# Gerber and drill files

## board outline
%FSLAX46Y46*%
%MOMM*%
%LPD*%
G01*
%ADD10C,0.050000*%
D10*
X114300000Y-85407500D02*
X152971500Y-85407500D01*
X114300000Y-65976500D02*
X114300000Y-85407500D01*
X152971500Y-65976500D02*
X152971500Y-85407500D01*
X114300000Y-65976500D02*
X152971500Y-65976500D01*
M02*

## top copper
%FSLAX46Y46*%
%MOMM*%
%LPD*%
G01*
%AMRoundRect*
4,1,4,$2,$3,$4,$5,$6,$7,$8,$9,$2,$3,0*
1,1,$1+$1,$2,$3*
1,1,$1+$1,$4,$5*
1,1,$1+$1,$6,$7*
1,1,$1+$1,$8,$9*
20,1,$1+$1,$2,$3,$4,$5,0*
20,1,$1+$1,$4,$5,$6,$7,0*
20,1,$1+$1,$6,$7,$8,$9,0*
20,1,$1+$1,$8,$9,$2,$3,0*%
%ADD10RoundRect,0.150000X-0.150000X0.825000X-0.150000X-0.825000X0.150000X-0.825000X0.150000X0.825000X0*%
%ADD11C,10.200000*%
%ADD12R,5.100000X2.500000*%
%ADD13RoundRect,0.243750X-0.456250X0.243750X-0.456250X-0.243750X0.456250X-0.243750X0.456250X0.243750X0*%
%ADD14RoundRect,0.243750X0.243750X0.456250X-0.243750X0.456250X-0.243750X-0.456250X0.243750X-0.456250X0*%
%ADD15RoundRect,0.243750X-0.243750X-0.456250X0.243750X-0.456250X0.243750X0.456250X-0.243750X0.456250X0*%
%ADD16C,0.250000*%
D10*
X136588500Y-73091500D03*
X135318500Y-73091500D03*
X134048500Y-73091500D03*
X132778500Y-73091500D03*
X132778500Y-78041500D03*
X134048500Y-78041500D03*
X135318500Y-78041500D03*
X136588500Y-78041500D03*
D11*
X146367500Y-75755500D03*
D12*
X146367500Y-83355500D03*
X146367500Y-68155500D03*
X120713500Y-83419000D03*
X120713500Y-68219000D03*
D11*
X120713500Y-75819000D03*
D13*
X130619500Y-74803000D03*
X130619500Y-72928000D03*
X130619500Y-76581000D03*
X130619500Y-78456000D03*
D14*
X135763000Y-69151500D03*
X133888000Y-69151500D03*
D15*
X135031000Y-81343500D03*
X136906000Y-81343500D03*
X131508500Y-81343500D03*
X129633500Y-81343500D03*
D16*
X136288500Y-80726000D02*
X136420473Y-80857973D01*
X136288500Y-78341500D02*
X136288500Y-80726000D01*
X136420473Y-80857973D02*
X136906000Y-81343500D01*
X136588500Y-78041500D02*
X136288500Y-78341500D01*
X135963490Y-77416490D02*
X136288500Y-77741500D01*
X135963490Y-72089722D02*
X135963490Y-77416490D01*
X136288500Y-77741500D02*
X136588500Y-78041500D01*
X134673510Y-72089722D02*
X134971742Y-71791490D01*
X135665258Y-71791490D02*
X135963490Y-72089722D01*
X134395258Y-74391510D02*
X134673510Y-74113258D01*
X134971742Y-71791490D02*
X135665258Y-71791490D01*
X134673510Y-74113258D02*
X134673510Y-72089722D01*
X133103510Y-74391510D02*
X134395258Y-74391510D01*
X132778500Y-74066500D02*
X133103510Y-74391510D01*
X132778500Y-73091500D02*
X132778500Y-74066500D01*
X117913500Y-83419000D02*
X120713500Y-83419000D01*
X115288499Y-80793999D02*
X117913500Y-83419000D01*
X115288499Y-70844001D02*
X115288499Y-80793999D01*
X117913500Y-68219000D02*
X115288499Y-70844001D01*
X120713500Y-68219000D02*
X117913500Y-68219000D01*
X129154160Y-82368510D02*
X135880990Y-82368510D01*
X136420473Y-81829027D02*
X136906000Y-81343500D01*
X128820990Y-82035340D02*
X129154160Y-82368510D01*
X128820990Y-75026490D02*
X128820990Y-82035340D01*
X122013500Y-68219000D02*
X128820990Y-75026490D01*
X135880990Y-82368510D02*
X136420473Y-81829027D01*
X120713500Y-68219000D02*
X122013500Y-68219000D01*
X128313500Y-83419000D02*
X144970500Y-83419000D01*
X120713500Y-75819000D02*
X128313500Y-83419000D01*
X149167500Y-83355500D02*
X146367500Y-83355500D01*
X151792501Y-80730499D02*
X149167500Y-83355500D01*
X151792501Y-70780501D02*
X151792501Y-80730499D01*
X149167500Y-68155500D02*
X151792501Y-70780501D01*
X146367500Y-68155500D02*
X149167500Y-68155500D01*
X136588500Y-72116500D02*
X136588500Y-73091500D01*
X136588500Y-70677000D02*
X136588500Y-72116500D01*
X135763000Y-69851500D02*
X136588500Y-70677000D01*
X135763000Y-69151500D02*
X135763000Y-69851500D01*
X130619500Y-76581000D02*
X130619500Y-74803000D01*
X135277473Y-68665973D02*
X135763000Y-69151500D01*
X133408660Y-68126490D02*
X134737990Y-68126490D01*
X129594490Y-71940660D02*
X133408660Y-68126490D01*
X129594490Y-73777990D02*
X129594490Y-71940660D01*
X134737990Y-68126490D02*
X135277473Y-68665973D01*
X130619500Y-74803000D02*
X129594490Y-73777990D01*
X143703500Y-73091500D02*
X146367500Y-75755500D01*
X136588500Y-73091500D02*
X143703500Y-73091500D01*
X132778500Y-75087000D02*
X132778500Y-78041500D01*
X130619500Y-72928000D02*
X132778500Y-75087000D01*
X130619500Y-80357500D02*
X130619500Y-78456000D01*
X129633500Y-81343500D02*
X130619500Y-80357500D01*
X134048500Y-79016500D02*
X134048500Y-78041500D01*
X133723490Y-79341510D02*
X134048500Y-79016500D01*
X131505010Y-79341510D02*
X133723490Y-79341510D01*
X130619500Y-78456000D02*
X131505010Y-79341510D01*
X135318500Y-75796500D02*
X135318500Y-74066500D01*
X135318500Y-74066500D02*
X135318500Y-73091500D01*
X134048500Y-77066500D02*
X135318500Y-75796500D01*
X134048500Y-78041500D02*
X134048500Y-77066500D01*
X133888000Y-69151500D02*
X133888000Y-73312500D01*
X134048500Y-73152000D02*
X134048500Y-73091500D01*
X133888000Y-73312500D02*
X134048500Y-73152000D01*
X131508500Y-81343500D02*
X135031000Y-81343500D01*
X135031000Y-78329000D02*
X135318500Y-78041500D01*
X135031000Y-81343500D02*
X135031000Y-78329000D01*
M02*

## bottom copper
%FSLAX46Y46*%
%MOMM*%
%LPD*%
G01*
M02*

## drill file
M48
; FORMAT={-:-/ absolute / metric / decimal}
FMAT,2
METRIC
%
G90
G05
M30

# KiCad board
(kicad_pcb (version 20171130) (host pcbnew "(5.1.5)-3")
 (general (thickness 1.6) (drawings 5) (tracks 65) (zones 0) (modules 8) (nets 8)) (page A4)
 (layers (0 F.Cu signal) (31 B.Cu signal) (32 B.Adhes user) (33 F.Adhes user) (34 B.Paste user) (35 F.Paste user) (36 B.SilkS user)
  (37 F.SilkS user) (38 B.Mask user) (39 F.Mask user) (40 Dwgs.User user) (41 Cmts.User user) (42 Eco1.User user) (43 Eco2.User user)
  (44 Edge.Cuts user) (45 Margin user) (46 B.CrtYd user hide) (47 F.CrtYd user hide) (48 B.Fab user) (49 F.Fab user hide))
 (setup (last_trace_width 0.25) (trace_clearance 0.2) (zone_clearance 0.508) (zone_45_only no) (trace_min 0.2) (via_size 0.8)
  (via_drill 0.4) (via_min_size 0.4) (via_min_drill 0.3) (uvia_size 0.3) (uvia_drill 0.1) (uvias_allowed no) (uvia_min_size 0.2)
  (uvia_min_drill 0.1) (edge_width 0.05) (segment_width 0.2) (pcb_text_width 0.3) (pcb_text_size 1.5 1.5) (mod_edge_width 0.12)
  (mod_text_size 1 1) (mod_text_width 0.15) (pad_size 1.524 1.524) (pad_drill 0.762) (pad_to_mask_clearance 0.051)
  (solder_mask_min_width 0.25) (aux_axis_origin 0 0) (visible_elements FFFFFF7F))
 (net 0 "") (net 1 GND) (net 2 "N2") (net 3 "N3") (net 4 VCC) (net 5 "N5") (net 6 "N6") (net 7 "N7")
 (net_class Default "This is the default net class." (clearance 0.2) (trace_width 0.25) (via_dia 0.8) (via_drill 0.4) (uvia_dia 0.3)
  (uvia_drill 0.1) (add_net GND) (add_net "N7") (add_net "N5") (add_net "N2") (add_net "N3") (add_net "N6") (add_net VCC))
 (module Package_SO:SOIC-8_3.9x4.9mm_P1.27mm (layer F.Cu) (at 134.6835 75.5665 270)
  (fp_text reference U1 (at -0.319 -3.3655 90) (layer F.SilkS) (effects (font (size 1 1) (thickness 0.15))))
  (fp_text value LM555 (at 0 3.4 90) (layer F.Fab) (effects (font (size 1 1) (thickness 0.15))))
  (pad 1 smd roundrect (at -2.475 -1.905 270) (size 1.95 0.6) (layers F.Cu F.Paste F.Mask) (roundrect_rratio 0.25) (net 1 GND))
  (pad 2 smd roundrect (at -2.475 -0.635 270) (size 1.95 0.6) (layers F.Cu F.Paste F.Mask) (roundrect_rratio 0.25) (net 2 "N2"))
  (pad 3 smd roundrect (at -2.475 0.635 270) (size 1.95 0.6) (layers F.Cu F.Paste F.Mask) (roundrect_rratio 0.25) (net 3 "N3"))
  (pad 4 smd roundrect (at -2.475 1.905 270) (size 1.95 0.6) (layers F.Cu F.Paste F.Mask) (roundrect_rratio 0.25) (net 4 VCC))
  (pad 5 smd roundrect (at 2.475 1.905 270) (size 1.95 0.6) (layers F.Cu F.Paste F.Mask) (roundrect_rratio 0.25) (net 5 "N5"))
  (pad 6 smd roundrect (at 2.475 0.635 270) (size 1.95 0.6) (layers F.Cu F.Paste F.Mask) (roundrect_rratio 0.25) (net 2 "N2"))
  (pad 7 smd roundrect (at 2.475 -0.635 270) (size 1.95 0.6) (layers F.Cu F.Paste F.Mask) (roundrect_rratio 0.25) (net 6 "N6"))
  (pad 8 smd roundrect (at 2.475 -1.905 270) (size 1.95 0.6) (layers F.Cu F.Paste F.Mask) (roundrect_rratio 0.25) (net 4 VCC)))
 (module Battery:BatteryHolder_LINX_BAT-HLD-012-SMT (layer F.Cu) (at 146.3675 75.7555 270)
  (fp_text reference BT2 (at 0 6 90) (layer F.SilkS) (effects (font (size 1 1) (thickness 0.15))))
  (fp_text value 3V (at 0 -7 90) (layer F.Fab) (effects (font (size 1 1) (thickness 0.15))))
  (pad 2 smd circle (at 0 0 270) (size 10.2 10.2) (layers F.Cu F.Mask) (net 1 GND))
  (pad 1 smd rect (at 7.6 0 270) (size 2.5 5.1) (layers F.Cu F.Paste F.Mask) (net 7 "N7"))
  (pad 1 smd rect (at -7.6 0 270) (size 2.5 5.1) (layers F.Cu F.Paste F.Mask) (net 7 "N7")))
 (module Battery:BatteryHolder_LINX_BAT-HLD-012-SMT (layer F.Cu) (at 120.7135 75.819 90)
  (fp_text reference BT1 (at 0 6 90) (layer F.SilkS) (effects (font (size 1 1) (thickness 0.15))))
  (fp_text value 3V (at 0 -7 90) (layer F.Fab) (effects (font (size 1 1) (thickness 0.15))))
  (pad 1 smd rect (at -7.6 0 90) (size 2.5 5.1) (layers F.Cu F.Paste F.Mask) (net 4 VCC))
  (pad 1 smd rect (at 7.6 0 90) (size 2.5 5.1) (layers F.Cu F.Paste F.Mask) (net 4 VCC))
  (pad 2 smd circle (at 0 0 90) (size 10.2 10.2) (layers F.Cu F.Mask) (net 7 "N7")))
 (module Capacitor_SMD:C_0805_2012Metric (layer F.Cu) (at 130.6195 73.8655 270)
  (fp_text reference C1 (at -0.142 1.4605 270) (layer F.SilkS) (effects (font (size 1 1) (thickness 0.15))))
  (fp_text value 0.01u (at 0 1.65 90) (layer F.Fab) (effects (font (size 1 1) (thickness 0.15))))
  (pad 2 smd roundrect (at 0.9375 0 270) (size 0.975 1.4) (layers F.Cu F.Paste F.Mask) (roundrect_rratio 0.25) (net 1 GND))
  (pad 1 smd roundrect (at -0.9375 0 270) (size 0.975 1.4) (layers F.Cu F.Paste F.Mask) (roundrect_rratio 0.25) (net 5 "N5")))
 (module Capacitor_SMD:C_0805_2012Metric (layer F.Cu) (at 130.6195 77.5185 270)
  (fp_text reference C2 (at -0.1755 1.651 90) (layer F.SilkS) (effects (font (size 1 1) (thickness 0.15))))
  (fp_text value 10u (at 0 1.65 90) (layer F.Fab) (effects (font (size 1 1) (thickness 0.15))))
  (pad 1 smd roundrect (at -0.9375 0 270) (size 0.975 1.4) (layers F.Cu F.Paste F.Mask) (roundrect_rratio 0.25) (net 1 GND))
  (pad 2 smd roundrect (at 0.9375 0 270) (size 0.975 1.4) (layers F.Cu F.Paste F.Mask) (roundrect_rratio 0.25) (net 2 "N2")))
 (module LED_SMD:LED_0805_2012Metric (layer F.Cu) (at 134.8255 69.1515 180)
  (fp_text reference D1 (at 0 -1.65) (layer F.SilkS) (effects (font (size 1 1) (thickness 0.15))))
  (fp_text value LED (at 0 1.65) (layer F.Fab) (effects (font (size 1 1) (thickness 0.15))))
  (pad 1 smd roundrect (at -0.9375 0 180) (size 0.975 1.4) (layers F.Cu F.Paste F.Mask) (roundrect_rratio 0.25) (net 1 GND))
  (pad 2 smd roundrect (at 0.9375 0 180) (size 0.975 1.4) (layers F.Cu F.Paste F.Mask) (roundrect_rratio 0.25) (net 3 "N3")))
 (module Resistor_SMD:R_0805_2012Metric (layer F.Cu) (at 135.9685 81.3435)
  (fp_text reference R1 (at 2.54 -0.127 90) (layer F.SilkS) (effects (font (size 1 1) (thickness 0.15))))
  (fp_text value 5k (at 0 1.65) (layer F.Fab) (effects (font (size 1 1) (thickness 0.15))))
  (pad 1 smd roundrect (at -0.9375 0) (size 0.975 1.4) (layers F.Cu F.Paste F.Mask) (roundrect_rratio 0.25) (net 6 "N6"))
  (pad 2 smd roundrect (at 0.9375 0) (size 0.975 1.4) (layers F.Cu F.Paste F.Mask) (roundrect_rratio 0.25) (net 4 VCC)))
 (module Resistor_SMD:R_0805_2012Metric (layer F.Cu) (at 130.571 81.3435)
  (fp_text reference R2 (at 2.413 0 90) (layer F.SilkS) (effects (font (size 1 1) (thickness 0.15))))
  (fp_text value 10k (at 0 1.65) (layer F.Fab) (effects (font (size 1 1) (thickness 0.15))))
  (pad 2 smd roundrect (at 0.9375 0) (size 0.975 1.4) (layers F.Cu F.Paste F.Mask) (roundrect_rratio 0.25) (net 6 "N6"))
  (pad 1 smd roundrect (at -0.9375 0) (size 0.975 1.4) (layers F.Cu F.Paste F.Mask) (roundrect_rratio 0.25) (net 2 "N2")))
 (gr_line (start 114.3 85.4075) (end 152.9715 85.4075) (layer Edge.Cuts) (width 0.05))
 (gr_line (start 114.3 65.9765) (end 114.3 85.4075) (layer Edge.Cuts) (width 0.05))
 (gr_line (start 152.9715 65.9765) (end 152.9715 85.4075) (layer Edge.Cuts) (width 0.05))
 (gr_line (start 114.3 65.9765) (end 152.9715 65.9765) (layer Edge.Cuts) (width 0.05))
 (segment (start 136.2885 80.726) (end 136.420473 80.857973) (width 0.25) (layer F.Cu) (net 4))
 (segment (start 136.2885 78.3415) (end 136.2885 80.726) (width 0.25) (layer F.Cu) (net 4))
 (segment (start 136.420473 80.857973) (end 136.906 81.3435) (width 0.25) (layer F.Cu) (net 4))
 (segment (start 136.5885 78.0415) (end 136.2885 78.3415) (width 0.25) (layer F.Cu) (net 4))
 (segment (start 135.96349 77.41649) (end 136.2885 77.7415) (width 0.25) (layer F.Cu) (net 4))
 (segment (start 135.96349 72.089722) (end 135.96349 77.41649) (width 0.25) (layer F.Cu) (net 4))
 (segment (start 136.2885 77.7415) (end 136.5885 78.0415) (width 0.25) (layer F.Cu) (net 4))
 (segment (start 134.67351 72.089722) (end 134.971742 71.79149) (width 0.25) (layer F.Cu) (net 4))
 (segment (start 135.665258 71.79149) (end 135.96349 72.089722) (width 0.25) (layer F.Cu) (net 4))
 (segment (start 134.395258 74.39151) (end 134.67351 74.113258) (width 0.25) (layer F.Cu) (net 4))
 (segment (start 134.971742 71.79149) (end 135.665258 71.79149) (width 0.25) (layer F.Cu) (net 4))
 (segment (start 134.67351 74.113258) (end 134.67351 72.089722) (width 0.25) (layer F.Cu) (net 4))
 (segment (start 133.10351 74.39151) (end 134.395258 74.39151) (width 0.25) (layer F.Cu) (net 4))
 (segment (start 132.7785 74.0665) (end 133.10351 74.39151) (width 0.25) (layer F.Cu) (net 4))
 (segment (start 132.7785 73.0915) (end 132.7785 74.0665) (width 0.25) (layer F.Cu) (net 4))
 (segment (start 117.9135 83.419) (end 120.7135 83.419) (width 0.25) (layer F.Cu) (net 4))
 (segment (start 115.288499 80.793999) (end 117.9135 83.419) (width 0.25) (layer F.Cu) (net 4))
 (segment (start 115.288499 70.844001) (end 115.288499 80.793999) (width 0.25) (layer F.Cu) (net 4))
 (segment (start 117.9135 68.219) (end 115.288499 70.844001) (width 0.25) (layer F.Cu) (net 4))
 (segment (start 120.7135 68.219) (end 117.9135 68.219) (width 0.25) (layer F.Cu) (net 4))
 (segment (start 129.15416 82.36851) (end 135.88099 82.36851) (width 0.25) (layer F.Cu) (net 4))
 (segment (start 136.420473 81.829027) (end 136.906 81.3435) (width 0.25) (layer F.Cu) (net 4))
 (segment (start 128.82099 82.03534) (end 129.15416 82.36851) (width 0.25) (layer F.Cu) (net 4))
 (segment (start 128.82099 75.02649) (end 128.82099 82.03534) (width 0.25) (layer F.Cu) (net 4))
 (segment (start 122.0135 68.219) (end 128.82099 75.02649) (width 0.25) (layer F.Cu) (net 4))
 (segment (start 135.88099 82.36851) (end 136.420473 81.829027) (width 0.25) (layer F.Cu) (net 4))
 (segment (start 120.7135 68.219) (end 122.0135 68.219) (width 0.25) (layer F.Cu) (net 4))
 (segment (start 128.3135 83.419) (end 144.9705 83.419) (width 0.25) (layer F.Cu) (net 7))
 (segment (start 120.7135 75.819) (end 128.3135 83.419) (width 0.25) (layer F.Cu) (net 7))
 (segment (start 149.1675 83.3555) (end 146.3675 83.3555) (width 0.25) (layer F.Cu) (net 7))
 (segment (start 151.792501 80.730499) (end 149.1675 83.3555) (width 0.25) (layer F.Cu) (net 7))
 (segment (start 151.792501 70.780501) (end 151.792501 80.730499) (width 0.25) (layer F.Cu) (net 7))
 (segment (start 149.1675 68.1555) (end 151.792501 70.780501) (width 0.25) (layer F.Cu) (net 7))
 (segment (start 146.3675 68.1555) (end 149.1675 68.1555) (width 0.25) (layer F.Cu) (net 7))
 (segment (start 136.5885 72.1165) (end 136.5885 73.0915) (width 0.25) (layer F.Cu) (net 1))
 (segment (start 136.5885 70.677) (end 136.5885 72.1165) (width 0.25) (layer F.Cu) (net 1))
 (segment (start 135.763 69.8515) (end 136.5885 70.677) (width 0.25) (layer F.Cu) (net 1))
 (segment (start 135.763 69.1515) (end 135.763 69.8515) (width 0.25) (layer F.Cu) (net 1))
 (segment (start 130.6195 76.581) (end 130.6195 74.803) (width 0.25) (layer F.Cu) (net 1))
 (segment (start 135.277473 68.665973) (end 135.763 69.1515) (width 0.25) (layer F.Cu) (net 1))
 (segment (start 133.40866 68.12649) (end 134.73799 68.12649) (width 0.25) (layer F.Cu) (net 1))
 (segment (start 129.59449 71.94066) (end 133.40866 68.12649) (width 0.25) (layer F.Cu) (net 1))
 (segment (start 129.59449 73.77799) (end 129.59449 71.94066) (width 0.25) (layer F.Cu) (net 1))
 (segment (start 134.73799 68.12649) (end 135.277473 68.665973) (width 0.25) (layer F.Cu) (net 1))
 (segment (start 130.6195 74.803) (end 129.59449 73.77799) (width 0.25) (layer F.Cu) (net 1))
 (segment (start 143.7035 73.0915) (end 146.3675 75.7555) (width 0.25) (layer F.Cu) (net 1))
 (segment (start 136.5885 73.0915) (end 143.7035 73.0915) (width 0.25) (layer F.Cu) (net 1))
 (segment (start 132.7785 75.087) (end 132.7785 78.0415) (width 0.25) (layer F.Cu) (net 5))
 (segment (start 130.6195 72.928) (end 132.7785 75.087) (width 0.25) (layer F.Cu) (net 5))
 (segment (start 130.6195 80.3575) (end 130.6195 78.456) (width 0.25) (layer F.Cu) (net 2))
 (segment (start 129.6335 81.3435) (end 130.6195 80.3575) (width 0.25) (layer F.Cu) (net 2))
 (segment (start 134.0485 79.0165) (end 134.0485 78.0415) (width 0.25) (layer F.Cu) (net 2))
 (segment (start 133.72349 79.34151) (end 134.0485 79.0165) (width 0.25) (layer F.Cu) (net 2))
 (segment (start 131.50501 79.34151) (end 133.72349 79.34151) (width 0.25) (layer F.Cu) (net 2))
 (segment (start 130.6195 78.456) (end 131.50501 79.34151) (width 0.25) (layer F.Cu) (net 2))
 (segment (start 135.3185 75.7965) (end 135.3185 74.0665) (width 0.25) (layer F.Cu) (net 2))
 (segment (start 135.3185 74.0665) (end 135.3185 73.0915) (width 0.25) (layer F.Cu) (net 2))
 (segment (start 134.0485 77.0665) (end 135.3185 75.7965) (width 0.25) (layer F.Cu) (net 2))
 (segment (start 134.0485 78.0415) (end 134.0485 77.0665) (width 0.25) (layer F.Cu) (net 2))
 (segment (start 133.888 69.1515) (end 133.888 73.3125) (width 0.25) (layer F.Cu) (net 3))
 (segment (start 134.0485 73.152) (end 134.0485 73.0915) (width 0.25) (layer F.Cu) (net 3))
 (segment (start 133.888 73.3125) (end 134.0485 73.152) (width 0.25) (layer F.Cu) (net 3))
 (segment (start 131.5085 81.3435) (end 135.031 81.3435) (width 0.25) (layer F.Cu) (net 6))
 (segment (start 135.031 78.329) (end 135.3185 78.0415) (width 0.25) (layer F.Cu) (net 6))
 (segment (start 135.031 81.3435) (end 135.031 78.329) (width 0.25) (layer F.Cu) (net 6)))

